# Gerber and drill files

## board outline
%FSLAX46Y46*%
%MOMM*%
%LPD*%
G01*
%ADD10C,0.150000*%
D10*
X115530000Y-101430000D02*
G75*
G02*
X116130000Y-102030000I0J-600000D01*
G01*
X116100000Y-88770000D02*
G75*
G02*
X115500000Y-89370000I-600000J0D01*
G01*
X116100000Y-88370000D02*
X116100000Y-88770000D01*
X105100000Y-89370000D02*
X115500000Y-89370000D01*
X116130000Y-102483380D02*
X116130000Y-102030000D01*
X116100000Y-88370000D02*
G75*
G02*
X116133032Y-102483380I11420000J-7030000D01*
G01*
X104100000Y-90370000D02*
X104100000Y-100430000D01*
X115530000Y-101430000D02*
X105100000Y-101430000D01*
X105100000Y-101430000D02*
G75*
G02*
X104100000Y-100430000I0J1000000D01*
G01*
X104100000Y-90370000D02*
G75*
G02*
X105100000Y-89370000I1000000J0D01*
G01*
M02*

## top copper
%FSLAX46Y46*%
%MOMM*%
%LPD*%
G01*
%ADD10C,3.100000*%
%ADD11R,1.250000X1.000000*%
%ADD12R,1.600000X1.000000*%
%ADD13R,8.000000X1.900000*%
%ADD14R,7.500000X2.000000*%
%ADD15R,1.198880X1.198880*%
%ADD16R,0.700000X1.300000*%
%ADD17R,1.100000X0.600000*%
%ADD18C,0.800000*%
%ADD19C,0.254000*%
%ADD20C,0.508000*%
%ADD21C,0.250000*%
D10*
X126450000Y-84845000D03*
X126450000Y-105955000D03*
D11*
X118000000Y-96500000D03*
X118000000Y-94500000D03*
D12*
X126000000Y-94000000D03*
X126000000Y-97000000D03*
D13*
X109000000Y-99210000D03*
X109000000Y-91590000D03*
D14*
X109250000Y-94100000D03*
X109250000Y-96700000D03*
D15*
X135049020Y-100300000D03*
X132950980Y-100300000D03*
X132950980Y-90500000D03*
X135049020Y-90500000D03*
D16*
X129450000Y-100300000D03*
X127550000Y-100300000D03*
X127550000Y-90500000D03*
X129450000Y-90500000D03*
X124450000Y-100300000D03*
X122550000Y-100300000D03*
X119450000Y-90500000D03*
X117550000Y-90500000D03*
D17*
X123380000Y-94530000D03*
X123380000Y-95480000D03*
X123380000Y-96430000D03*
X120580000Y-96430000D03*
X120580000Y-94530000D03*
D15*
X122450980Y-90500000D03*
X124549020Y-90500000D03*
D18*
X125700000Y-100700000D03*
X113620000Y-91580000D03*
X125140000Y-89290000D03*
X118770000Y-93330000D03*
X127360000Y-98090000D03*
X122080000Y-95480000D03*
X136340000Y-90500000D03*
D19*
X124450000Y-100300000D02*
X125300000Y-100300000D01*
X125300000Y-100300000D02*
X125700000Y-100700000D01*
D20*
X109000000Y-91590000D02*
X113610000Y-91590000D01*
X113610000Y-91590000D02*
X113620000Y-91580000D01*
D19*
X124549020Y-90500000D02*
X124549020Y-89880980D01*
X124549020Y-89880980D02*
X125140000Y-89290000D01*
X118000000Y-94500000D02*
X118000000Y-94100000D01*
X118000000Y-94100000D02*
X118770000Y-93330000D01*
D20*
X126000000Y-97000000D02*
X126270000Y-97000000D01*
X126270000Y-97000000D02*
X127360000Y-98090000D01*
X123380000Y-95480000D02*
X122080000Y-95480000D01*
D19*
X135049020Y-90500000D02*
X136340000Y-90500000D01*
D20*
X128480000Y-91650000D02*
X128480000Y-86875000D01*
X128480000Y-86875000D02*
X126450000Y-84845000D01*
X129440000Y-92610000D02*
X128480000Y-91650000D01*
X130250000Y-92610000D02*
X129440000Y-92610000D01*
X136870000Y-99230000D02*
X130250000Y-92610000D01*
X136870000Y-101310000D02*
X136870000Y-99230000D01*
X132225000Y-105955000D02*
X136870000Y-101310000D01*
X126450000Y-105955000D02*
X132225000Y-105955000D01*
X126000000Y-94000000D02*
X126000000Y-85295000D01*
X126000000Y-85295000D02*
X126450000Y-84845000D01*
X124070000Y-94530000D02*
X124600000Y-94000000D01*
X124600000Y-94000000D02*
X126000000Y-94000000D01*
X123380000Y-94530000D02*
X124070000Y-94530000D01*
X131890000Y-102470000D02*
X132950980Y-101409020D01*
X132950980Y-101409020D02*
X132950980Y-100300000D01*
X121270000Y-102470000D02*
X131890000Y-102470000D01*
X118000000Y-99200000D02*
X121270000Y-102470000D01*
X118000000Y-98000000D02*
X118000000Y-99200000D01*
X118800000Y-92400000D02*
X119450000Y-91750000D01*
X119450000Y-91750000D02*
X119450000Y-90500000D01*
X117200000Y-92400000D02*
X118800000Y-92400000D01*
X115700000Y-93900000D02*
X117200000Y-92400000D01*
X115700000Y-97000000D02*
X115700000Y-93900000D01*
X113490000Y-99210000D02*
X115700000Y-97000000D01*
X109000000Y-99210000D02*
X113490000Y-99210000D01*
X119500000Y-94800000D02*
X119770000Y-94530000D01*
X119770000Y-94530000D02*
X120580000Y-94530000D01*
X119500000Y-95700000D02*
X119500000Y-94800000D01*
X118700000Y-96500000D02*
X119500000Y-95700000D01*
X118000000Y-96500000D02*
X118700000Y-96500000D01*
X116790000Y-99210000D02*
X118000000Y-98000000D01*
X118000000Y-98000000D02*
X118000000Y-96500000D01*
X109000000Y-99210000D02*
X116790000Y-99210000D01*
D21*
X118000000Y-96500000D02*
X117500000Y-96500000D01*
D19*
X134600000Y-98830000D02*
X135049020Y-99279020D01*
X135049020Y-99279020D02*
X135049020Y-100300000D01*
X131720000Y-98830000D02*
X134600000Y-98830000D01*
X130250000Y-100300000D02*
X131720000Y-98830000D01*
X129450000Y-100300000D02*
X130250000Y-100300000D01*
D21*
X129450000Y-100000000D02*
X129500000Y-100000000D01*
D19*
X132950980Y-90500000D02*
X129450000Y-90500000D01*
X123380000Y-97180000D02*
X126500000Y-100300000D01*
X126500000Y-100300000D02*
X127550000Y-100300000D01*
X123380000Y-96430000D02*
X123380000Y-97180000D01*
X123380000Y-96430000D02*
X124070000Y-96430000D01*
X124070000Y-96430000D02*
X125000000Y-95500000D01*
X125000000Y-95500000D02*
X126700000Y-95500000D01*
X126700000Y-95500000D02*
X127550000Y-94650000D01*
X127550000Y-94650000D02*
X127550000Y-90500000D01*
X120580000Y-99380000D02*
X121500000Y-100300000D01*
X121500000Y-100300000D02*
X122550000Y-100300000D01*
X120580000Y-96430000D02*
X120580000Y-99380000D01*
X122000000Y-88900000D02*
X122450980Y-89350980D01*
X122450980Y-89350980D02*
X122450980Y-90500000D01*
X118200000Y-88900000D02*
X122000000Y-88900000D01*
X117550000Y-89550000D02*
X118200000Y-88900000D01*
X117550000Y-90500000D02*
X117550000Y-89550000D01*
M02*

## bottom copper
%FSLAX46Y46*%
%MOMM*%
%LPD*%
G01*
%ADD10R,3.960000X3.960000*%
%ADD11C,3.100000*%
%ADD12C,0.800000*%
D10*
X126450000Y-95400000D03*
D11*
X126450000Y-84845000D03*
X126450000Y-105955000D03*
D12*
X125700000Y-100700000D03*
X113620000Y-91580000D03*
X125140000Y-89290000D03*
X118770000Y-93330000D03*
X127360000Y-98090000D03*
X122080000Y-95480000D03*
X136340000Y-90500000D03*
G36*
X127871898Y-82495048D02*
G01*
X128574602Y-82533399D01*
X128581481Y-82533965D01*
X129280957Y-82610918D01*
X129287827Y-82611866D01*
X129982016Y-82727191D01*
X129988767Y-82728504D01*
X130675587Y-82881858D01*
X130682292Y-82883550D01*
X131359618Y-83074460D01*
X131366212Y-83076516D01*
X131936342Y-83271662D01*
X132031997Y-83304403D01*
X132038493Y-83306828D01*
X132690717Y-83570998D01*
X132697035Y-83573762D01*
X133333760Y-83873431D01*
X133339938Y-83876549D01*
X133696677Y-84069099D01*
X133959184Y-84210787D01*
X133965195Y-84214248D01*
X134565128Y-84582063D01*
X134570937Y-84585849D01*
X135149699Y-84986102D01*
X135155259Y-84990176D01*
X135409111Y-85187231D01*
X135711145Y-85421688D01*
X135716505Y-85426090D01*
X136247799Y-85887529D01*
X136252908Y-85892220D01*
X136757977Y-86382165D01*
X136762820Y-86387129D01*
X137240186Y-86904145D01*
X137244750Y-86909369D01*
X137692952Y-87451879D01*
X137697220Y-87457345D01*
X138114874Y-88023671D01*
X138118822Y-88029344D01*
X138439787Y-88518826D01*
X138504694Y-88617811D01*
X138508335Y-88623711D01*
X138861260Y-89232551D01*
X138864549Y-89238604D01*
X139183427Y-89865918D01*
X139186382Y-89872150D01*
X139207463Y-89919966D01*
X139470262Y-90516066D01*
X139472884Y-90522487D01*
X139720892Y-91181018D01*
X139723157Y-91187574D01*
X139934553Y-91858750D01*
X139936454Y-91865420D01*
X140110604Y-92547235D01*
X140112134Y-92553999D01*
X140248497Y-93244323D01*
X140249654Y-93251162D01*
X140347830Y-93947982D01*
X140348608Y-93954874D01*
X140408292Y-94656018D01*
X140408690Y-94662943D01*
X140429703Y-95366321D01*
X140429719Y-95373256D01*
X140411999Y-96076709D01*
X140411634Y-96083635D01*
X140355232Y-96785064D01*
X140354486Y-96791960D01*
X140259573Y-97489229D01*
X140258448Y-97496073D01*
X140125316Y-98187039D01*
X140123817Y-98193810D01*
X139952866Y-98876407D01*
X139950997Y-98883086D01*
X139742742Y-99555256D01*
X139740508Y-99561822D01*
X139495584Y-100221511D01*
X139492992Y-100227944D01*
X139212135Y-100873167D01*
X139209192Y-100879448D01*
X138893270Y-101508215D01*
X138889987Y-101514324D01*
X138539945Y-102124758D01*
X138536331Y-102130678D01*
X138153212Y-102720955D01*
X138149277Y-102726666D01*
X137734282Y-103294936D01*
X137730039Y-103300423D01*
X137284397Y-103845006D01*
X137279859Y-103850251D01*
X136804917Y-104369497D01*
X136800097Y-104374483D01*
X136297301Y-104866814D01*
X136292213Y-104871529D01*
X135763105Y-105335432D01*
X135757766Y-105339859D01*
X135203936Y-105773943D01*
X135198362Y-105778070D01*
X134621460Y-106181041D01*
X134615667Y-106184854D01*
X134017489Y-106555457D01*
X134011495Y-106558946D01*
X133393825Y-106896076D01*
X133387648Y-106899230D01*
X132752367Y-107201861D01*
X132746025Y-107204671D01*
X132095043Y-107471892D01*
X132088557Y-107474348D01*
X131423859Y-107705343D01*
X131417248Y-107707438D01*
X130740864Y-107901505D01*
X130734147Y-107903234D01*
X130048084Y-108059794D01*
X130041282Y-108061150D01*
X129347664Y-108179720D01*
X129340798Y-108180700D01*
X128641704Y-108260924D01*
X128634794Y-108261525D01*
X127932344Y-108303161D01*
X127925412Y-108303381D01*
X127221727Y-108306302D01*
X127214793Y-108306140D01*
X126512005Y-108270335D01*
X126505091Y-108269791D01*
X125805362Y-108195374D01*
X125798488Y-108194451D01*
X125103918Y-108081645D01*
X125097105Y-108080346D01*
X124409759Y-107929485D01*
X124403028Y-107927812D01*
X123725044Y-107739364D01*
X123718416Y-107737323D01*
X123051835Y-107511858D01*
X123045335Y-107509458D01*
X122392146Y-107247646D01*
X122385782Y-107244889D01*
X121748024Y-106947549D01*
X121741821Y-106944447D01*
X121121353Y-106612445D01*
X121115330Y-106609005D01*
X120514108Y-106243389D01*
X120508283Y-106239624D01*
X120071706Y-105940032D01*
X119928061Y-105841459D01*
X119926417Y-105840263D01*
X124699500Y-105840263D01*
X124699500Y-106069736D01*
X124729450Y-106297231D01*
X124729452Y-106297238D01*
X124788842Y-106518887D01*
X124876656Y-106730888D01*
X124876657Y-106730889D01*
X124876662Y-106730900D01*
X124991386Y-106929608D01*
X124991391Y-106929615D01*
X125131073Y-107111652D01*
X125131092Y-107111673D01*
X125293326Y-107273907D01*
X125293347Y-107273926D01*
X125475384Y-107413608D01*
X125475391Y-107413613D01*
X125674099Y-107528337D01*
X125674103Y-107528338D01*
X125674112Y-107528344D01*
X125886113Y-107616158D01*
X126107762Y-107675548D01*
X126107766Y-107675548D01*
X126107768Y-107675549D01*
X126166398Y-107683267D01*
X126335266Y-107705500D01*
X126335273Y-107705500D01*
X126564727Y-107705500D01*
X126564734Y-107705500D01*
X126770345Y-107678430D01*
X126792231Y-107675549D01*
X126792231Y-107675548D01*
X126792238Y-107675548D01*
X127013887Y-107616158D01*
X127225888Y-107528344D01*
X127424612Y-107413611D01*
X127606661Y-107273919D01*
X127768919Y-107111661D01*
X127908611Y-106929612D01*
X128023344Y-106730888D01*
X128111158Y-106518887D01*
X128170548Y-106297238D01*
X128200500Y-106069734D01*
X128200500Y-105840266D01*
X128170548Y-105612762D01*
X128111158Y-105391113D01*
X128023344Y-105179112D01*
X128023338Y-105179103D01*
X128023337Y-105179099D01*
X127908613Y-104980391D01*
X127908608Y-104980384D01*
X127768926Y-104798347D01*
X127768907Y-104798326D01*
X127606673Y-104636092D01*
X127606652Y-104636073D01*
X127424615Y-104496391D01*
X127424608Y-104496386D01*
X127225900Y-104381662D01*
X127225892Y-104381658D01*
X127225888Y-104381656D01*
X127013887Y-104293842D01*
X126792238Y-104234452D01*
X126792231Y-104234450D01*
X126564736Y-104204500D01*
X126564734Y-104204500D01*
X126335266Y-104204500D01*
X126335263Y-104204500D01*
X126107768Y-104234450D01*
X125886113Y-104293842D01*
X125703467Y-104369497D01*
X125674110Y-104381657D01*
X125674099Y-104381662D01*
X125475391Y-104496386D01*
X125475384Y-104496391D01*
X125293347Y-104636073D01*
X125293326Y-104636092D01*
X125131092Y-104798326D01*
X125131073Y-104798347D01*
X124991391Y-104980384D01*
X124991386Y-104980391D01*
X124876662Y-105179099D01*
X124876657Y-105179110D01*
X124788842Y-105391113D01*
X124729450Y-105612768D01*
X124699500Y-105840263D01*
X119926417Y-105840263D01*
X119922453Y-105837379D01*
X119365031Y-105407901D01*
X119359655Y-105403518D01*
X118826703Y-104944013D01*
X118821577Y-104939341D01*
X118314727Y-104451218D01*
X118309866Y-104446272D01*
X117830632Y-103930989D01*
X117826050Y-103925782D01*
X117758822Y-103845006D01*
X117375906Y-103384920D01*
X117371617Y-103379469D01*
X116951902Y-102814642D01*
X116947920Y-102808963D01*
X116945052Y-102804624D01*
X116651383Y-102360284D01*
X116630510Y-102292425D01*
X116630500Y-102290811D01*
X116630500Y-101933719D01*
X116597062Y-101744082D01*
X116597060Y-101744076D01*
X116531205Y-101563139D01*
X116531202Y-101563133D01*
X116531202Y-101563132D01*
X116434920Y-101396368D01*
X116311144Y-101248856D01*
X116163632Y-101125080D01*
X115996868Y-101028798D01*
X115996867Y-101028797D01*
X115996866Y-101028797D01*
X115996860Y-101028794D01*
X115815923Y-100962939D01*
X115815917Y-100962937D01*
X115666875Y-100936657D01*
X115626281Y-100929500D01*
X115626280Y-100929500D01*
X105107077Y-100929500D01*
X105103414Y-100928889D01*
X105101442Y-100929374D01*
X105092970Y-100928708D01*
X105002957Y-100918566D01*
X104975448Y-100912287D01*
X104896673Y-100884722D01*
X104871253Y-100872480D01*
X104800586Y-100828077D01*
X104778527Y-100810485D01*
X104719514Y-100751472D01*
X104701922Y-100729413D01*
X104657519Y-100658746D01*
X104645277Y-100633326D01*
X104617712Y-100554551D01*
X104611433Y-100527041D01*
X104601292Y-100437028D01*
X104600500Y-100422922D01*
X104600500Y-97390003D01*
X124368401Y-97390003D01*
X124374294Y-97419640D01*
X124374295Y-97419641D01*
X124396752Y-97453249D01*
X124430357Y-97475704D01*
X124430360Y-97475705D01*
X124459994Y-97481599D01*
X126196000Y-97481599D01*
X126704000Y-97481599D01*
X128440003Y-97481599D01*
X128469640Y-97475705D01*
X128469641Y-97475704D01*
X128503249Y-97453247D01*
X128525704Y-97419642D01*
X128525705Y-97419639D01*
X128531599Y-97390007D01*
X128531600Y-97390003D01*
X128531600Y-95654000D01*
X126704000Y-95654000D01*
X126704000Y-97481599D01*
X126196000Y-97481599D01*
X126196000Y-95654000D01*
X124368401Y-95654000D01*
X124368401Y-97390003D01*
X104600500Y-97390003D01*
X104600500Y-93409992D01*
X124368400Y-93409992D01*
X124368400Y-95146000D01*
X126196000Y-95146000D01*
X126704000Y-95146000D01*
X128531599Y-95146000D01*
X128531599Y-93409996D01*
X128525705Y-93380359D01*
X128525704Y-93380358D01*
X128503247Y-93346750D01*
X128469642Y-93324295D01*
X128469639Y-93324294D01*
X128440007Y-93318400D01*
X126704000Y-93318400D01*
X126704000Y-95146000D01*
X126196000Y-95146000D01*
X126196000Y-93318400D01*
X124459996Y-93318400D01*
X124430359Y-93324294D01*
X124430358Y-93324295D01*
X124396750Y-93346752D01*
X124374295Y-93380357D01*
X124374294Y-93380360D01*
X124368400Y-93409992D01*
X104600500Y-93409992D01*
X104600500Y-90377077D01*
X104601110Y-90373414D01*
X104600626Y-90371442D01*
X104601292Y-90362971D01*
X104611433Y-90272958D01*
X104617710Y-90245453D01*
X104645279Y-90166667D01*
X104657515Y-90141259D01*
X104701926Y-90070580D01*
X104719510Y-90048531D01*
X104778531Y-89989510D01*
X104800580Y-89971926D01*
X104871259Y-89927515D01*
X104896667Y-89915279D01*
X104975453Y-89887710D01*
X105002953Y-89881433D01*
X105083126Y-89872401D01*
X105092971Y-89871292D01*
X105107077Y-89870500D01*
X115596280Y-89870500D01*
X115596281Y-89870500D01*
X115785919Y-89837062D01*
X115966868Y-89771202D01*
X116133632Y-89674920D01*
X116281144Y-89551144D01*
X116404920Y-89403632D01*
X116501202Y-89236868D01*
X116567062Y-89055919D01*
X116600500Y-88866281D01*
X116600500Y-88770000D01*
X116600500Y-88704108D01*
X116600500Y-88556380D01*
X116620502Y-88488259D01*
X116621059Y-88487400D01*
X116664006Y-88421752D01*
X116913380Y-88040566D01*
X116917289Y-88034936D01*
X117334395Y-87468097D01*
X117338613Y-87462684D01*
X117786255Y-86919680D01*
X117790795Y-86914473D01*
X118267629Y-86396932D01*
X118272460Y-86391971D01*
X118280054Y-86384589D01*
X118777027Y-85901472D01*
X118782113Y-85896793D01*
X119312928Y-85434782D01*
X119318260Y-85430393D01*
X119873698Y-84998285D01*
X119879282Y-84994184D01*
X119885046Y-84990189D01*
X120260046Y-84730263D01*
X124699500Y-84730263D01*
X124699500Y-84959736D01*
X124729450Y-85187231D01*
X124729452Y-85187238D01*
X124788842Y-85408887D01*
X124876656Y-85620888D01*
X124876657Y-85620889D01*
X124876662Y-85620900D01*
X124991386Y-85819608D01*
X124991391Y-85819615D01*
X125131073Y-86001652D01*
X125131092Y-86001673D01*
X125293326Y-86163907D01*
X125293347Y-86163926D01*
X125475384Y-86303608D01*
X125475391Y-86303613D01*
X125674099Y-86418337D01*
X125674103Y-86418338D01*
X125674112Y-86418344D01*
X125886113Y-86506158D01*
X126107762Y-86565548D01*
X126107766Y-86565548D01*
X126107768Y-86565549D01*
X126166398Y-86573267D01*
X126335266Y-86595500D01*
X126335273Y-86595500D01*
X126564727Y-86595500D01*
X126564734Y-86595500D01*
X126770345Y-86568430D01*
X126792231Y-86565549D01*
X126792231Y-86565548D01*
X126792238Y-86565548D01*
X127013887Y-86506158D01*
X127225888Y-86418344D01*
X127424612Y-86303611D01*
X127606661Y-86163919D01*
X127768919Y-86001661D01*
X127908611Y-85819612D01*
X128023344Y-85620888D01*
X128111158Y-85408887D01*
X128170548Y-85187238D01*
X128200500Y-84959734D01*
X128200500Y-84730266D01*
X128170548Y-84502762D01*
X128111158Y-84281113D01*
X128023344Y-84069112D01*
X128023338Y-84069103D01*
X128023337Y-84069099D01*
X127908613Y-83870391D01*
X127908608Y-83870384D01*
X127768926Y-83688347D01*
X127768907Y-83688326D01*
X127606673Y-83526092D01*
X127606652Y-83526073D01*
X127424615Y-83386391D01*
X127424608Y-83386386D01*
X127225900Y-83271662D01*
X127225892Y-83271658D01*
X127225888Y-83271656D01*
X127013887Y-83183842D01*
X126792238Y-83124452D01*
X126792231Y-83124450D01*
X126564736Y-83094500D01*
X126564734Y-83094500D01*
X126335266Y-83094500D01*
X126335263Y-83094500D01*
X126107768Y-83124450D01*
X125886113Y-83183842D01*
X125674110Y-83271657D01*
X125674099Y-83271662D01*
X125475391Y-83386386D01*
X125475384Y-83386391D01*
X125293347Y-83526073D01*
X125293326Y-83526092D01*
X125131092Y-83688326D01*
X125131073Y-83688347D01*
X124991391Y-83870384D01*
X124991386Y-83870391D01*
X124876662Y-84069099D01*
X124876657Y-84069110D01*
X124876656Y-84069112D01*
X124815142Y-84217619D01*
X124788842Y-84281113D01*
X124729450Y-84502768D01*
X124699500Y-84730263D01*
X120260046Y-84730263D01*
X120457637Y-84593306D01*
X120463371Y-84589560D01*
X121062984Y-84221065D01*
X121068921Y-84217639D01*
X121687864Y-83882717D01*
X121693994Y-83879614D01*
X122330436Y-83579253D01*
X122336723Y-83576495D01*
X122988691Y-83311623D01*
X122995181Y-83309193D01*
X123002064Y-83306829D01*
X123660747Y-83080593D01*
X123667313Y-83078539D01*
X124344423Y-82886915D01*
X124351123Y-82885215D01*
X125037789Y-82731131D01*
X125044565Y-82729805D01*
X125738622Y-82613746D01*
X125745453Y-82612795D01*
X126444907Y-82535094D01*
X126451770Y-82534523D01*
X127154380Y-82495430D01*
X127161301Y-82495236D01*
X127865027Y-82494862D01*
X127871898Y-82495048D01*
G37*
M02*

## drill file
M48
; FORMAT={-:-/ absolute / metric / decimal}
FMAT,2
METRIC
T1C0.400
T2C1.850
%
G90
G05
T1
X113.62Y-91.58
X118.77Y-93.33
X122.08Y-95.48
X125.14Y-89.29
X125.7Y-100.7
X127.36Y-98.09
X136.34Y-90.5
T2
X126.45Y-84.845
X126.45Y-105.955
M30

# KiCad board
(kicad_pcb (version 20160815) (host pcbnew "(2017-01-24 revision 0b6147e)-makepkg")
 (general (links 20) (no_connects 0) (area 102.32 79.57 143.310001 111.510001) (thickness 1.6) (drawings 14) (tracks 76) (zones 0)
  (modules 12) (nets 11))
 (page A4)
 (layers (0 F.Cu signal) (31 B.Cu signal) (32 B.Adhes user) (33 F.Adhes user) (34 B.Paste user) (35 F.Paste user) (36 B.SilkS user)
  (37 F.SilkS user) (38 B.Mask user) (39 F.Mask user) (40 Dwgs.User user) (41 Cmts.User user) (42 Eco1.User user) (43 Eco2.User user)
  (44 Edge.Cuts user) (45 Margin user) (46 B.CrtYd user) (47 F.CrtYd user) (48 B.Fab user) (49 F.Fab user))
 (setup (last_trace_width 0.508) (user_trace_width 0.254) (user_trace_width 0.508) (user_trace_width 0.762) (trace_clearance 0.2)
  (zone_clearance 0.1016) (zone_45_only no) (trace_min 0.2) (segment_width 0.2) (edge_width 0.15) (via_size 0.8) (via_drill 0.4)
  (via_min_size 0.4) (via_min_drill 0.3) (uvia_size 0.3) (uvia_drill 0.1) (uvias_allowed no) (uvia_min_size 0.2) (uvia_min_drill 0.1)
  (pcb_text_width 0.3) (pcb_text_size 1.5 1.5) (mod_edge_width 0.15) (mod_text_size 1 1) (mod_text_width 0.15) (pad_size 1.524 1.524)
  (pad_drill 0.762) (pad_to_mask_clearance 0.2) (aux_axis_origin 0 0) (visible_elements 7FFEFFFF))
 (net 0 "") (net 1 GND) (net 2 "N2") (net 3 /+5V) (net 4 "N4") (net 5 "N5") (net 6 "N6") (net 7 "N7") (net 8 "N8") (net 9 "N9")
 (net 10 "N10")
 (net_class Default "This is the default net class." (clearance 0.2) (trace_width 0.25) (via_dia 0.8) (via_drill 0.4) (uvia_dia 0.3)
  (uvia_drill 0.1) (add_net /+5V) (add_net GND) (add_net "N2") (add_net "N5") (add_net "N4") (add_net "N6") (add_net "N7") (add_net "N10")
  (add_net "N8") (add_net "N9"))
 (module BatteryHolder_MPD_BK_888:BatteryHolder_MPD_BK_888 (layer B.Cu) (at 126.45 95.4 90)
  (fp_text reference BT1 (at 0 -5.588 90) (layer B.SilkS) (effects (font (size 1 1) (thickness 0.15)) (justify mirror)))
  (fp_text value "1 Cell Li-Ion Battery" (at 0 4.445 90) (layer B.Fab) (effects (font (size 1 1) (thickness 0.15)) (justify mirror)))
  (pad 2 smd rect (at 0 0 90) (size 3.96 3.96) (layers B.Cu B.Paste B.Mask) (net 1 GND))
  (pad 1 thru_hole circle (at 10.555 0 90) (size 3.1 3.1) (drill 1.85) (layers *.Cu *.Mask) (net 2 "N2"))
  (pad 1 thru_hole circle (at -10.555 0 90) (size 3.1 3.1) (drill 1.85) (layers *.Cu *.Mask) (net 2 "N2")))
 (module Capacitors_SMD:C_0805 (layer F.Cu) (at 118 95.5 90)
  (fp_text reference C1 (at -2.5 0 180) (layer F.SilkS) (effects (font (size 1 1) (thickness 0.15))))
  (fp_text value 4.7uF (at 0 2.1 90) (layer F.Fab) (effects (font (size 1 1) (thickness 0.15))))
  (pad 1 smd rect (at -1 0 90) (size 1 1.25) (layers F.Cu F.Paste F.Mask) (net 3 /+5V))
  (pad 2 smd rect (at 1 0 90) (size 1 1.25) (layers F.Cu F.Paste F.Mask) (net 1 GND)))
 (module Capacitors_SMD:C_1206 (layer F.Cu) (at 126 95.5 270)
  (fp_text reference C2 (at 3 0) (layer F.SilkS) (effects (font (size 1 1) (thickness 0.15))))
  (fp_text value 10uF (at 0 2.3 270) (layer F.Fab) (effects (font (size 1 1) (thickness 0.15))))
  (pad 1 smd rect (at -1.5 0 270) (size 1 1.6) (layers F.Cu F.Paste F.Mask) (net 2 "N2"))
  (pad 2 smd rect (at 1.5 0 270) (size 1 1.6) (layers F.Cu F.Paste F.Mask) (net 1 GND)))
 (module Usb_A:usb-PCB (layer F.Cu) (at 104.1 95.4 270)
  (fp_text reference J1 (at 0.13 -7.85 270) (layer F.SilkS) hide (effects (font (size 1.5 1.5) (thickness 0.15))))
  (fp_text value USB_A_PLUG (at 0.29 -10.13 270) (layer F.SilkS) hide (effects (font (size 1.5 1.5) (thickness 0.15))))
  (pad 1 connect rect (at 3.81 -4.9 270) (size 1.9 8) (layers F.Cu F.Mask) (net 3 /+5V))
  (pad 4 connect rect (at -3.81 -4.9 270) (size 1.9 8) (layers F.Cu F.Mask) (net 1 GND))
  (pad 3 connect rect (at -1.3 -5.15 270) (size 2 7.5) (layers F.Cu F.Mask) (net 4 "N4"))
  (pad 2 connect rect (at 1.3 -5.15 270) (size 2 7.5) (layers F.Cu F.Mask) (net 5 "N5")))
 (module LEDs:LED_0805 (layer F.Cu) (at 134 100.3 180)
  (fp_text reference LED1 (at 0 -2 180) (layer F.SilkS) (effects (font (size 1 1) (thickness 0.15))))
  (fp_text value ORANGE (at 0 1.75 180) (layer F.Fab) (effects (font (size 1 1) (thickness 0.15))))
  (pad 1 smd rect (at -1.04902 0) (size 1.19888 1.19888) (layers F.Cu F.Paste F.Mask) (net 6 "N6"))
  (pad 2 smd rect (at 1.04902 0) (size 1.19888 1.19888) (layers F.Cu F.Paste F.Mask) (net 3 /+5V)))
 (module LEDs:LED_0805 (layer F.Cu) (at 134 90.5 180)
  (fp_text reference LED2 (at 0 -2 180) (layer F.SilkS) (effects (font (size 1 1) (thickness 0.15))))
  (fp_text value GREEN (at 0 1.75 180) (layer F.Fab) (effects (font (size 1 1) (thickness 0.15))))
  (pad 2 smd rect (at 1.04902 0) (size 1.19888 1.19888) (layers F.Cu F.Paste F.Mask) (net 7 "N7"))
  (pad 1 smd rect (at -1.04902 0) (size 1.19888 1.19888) (layers F.Cu F.Paste F.Mask) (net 1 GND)))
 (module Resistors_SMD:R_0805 (layer F.Cu) (at 128.5 100.3 180)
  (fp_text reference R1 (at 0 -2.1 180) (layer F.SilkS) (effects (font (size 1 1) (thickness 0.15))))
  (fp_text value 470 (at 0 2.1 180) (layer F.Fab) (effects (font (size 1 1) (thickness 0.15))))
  (pad 1 smd rect (at -0.95 0 180) (size 0.7 1.3) (layers F.Cu F.Paste F.Mask) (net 6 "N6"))
  (pad 2 smd rect (at 0.95 0 180) (size 0.7 1.3) (layers F.Cu F.Paste F.Mask) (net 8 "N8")))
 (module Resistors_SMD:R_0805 (layer F.Cu) (at 128.5 90.5 180)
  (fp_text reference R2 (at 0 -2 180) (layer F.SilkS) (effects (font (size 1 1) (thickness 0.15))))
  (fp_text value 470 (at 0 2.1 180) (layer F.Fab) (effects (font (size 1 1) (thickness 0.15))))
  (pad 2 smd rect (at 0.95 0 180) (size 0.7 1.3) (layers F.Cu F.Paste F.Mask) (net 8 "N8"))
  (pad 1 smd rect (at -0.95 0 180) (size 0.7 1.3) (layers F.Cu F.Paste F.Mask) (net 7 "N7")))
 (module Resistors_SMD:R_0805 (layer F.Cu) (at 123.5 100.3)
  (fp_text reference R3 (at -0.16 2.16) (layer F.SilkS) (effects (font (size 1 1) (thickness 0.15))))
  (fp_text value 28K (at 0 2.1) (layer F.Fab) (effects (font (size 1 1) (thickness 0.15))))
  (pad 2 smd rect (at 0.95 0) (size 0.7 1.3) (layers F.Cu F.Paste F.Mask) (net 1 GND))
  (pad 1 smd rect (at -0.95 0) (size 0.7 1.3) (layers F.Cu F.Paste F.Mask) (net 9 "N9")))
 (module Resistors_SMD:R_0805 (layer F.Cu) (at 118.5 90.5 180)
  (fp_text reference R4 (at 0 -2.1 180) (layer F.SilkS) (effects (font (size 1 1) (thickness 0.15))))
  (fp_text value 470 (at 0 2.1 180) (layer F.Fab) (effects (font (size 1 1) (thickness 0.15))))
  (pad 1 smd rect (at -0.95 0 180) (size 0.7 1.3) (layers F.Cu F.Paste F.Mask) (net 3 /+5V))
  (pad 2 smd rect (at 0.95 0 180) (size 0.7 1.3) (layers F.Cu F.Paste F.Mask) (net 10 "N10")))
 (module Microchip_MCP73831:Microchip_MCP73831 (layer F.Cu) (at 122 95.5 90)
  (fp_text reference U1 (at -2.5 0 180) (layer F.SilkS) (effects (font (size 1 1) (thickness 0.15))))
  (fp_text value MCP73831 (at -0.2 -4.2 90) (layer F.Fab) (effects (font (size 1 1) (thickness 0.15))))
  (pad 3 smd rect (at 0.97 1.38 90) (size 0.6 1.1) (layers F.Cu F.Paste F.Mask) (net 2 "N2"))
  (pad 2 smd rect (at 0.02 1.38 90) (size 0.6 1.1) (layers F.Cu F.Paste F.Mask) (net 1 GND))
  (pad 1 smd rect (at -0.93 1.38 90) (size 0.6 1.1) (layers F.Cu F.Paste F.Mask) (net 8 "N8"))
  (pad 5 smd rect (at -0.93 -1.42 90) (size 0.6 1.1) (layers F.Cu F.Paste F.Mask) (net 9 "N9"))
  (pad 4 smd rect (at 0.97 -1.42 90) (size 0.6 1.1) (layers F.Cu F.Paste F.Mask) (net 3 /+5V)))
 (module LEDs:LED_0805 (layer F.Cu) (at 123.5 90.5 180)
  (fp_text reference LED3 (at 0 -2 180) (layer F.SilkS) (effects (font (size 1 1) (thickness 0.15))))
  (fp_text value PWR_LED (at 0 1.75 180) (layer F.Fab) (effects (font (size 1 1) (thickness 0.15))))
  (pad 2 smd rect (at 1.04902 0) (size 1.19888 1.19888) (layers F.Cu F.Paste F.Mask) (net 10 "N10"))
  (pad 1 smd rect (at -1.04902 0) (size 1.19888 1.19888) (layers F.Cu F.Paste F.Mask) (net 1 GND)))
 (gr_arc (start 115.53 102.03) (end 116.13 102.03) (angle -90) (layer Edge.Cuts) (width 0.15))
 (gr_arc (start 115.5 88.77) (end 116.1 88.77) (angle 90) (layer Edge.Cuts) (width 0.15))
 (gr_line (start 116.1 88.37) (end 116.1 88.77) (angle 90) (layer Edge.Cuts) (width 0.15))
 (gr_line (start 105.1 89.37) (end 115.5 89.37) (angle 90) (layer Edge.Cuts) (width 0.15))
 (gr_line (start 116.13 102.48338) (end 116.13 102.03) (angle 90) (layer Edge.Cuts) (width 0.15))
 (gr_arc (start 127.52 95.4) (end 116.1 88.37) (angle 296.5) (layer Edge.Cuts) (width 0.15))
 (gr_line (start 104.1 90.37) (end 104.1 100.43) (angle 90) (layer Edge.Cuts) (width 0.15))
 (gr_line (start 115.53 101.43) (end 105.1 101.43) (angle 90) (layer Edge.Cuts) (width 0.15))
 (gr_arc (start 105.1 100.43) (end 105.1 101.43) (angle 90) (layer Edge.Cuts) (width 0.15))
 (gr_arc (start 105.1 90.37) (end 104.1 90.37) (angle 90) (layer Edge.Cuts) (width 0.15))
 (segment (start 124.45 100.3) (end 125.3 100.3) (width 0.254) (layer F.Cu) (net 1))
 (segment (start 125.3 100.3) (end 125.7 100.7) (width 0.254) (layer F.Cu) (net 1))
 (via (at 125.7 100.7) (size 0.8) (drill 0.4) (layers F.Cu B.Cu) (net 1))
 (segment (start 109 91.59) (end 113.61 91.59) (width 0.508) (layer F.Cu) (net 1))
 (segment (start 113.61 91.59) (end 113.62 91.58) (width 0.508) (layer F.Cu) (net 1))
 (via (at 113.62 91.58) (size 0.8) (drill 0.4) (layers F.Cu B.Cu) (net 1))
 (segment (start 124.54902 90.5) (end 124.54902 89.88098) (width 0.254) (layer F.Cu) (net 1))
 (segment (start 124.54902 89.88098) (end 125.14 89.29) (width 0.254) (layer F.Cu) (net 1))
 (via (at 125.14 89.29) (size 0.8) (drill 0.4) (layers F.Cu B.Cu) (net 1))
 (segment (start 118 94.5) (end 118 94.1) (width 0.254) (layer F.Cu) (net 1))
 (segment (start 118 94.1) (end 118.77 93.33) (width 0.254) (layer F.Cu) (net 1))
 (via (at 118.77 93.33) (size 0.8) (drill 0.4) (layers F.Cu B.Cu) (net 1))
 (segment (start 126 97) (end 126.27 97) (width 0.508) (layer F.Cu) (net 1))
 (segment (start 126.27 97) (end 127.36 98.09) (width 0.508) (layer F.Cu) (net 1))
 (via (at 127.36 98.09) (size 0.8) (drill 0.4) (layers F.Cu B.Cu) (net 1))
 (segment (start 123.38 95.48) (end 122.08 95.48) (width 0.508) (layer F.Cu) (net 1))
 (via (at 122.08 95.48) (size 0.8) (drill 0.4) (layers F.Cu B.Cu) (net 1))
 (segment (start 135.04902 90.5) (end 136.34 90.5) (width 0.254) (layer F.Cu) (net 1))
 (via (at 136.34 90.5) (size 0.8) (drill 0.4) (layers F.Cu B.Cu) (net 1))
 (segment (start 128.48 91.65) (end 128.48 86.875) (width 0.508) (layer F.Cu) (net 2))
 (segment (start 128.48 86.875) (end 126.45 84.845) (width 0.508) (layer F.Cu) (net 2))
 (segment (start 129.44 92.61) (end 128.48 91.65) (width 0.508) (layer F.Cu) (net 2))
 (segment (start 130.25 92.61) (end 129.44 92.61) (width 0.508) (layer F.Cu) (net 2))
 (segment (start 136.87 99.23) (end 130.25 92.61) (width 0.508) (layer F.Cu) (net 2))
 (segment (start 136.87 101.31) (end 136.87 99.23) (width 0.508) (layer F.Cu) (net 2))
 (segment (start 132.225 105.955) (end 136.87 101.31) (width 0.508) (layer F.Cu) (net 2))
 (segment (start 126.45 105.955) (end 132.225 105.955) (width 0.508) (layer F.Cu) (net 2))
 (segment (start 126 94) (end 126 85.295) (width 0.508) (layer F.Cu) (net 2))
 (segment (start 126 85.295) (end 126.45 84.845) (width 0.508) (layer F.Cu) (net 2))
 (segment (start 124.07 94.53) (end 124.6 94) (width 0.508) (layer F.Cu) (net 2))
 (segment (start 124.6 94) (end 126 94) (width 0.508) (layer F.Cu) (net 2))
 (segment (start 123.38 94.53) (end 124.07 94.53) (width 0.508) (layer F.Cu) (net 2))
 (segment (start 131.89 102.47) (end 132.95098 101.40902) (width 0.508) (layer F.Cu) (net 3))
 (segment (start 132.95098 101.40902) (end 132.95098 100.3) (width 0.508) (layer F.Cu) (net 3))
 (segment (start 121.27 102.47) (end 131.89 102.47) (width 0.508) (layer F.Cu) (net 3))
 (segment (start 118 99.2) (end 121.27 102.47) (width 0.508) (layer F.Cu) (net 3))
 (segment (start 118 98) (end 118 99.2) (width 0.508) (layer F.Cu) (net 3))
 (segment (start 118.8 92.4) (end 119.45 91.75) (width 0.508) (layer F.Cu) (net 3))
 (segment (start 119.45 91.75) (end 119.45 90.5) (width 0.508) (layer F.Cu) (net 3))
 (segment (start 117.2 92.4) (end 118.8 92.4) (width 0.508) (layer F.Cu) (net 3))
 (segment (start 115.7 93.9) (end 117.2 92.4) (width 0.508) (layer F.Cu) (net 3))
 (segment (start 115.7 97) (end 115.7 93.9) (width 0.508) (layer F.Cu) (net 3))
 (segment (start 113.49 99.21) (end 115.7 97) (width 0.508) (layer F.Cu) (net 3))
 (segment (start 109 99.21) (end 113.49 99.21) (width 0.508) (layer F.Cu) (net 3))
 (segment (start 119.5 94.8) (end 119.77 94.53) (width 0.508) (layer F.Cu) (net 3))
 (segment (start 119.77 94.53) (end 120.58 94.53) (width 0.508) (layer F.Cu) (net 3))
 (segment (start 119.5 95.7) (end 119.5 94.8) (width 0.508) (layer F.Cu) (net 3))
 (segment (start 118.7 96.5) (end 119.5 95.7) (width 0.508) (layer F.Cu) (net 3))
 (segment (start 118 96.5) (end 118.7 96.5) (width 0.508) (layer F.Cu) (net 3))
 (segment (start 116.79 99.21) (end 118 98) (width 0.508) (layer F.Cu) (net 3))
 (segment (start 118 98) (end 118 96.5) (width 0.508) (layer F.Cu) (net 3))
 (segment (start 109 99.21) (end 116.79 99.21) (width 0.508) (layer F.Cu) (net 3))
 (segment (start 118 96.5) (end 117.5 96.5) (width 0.25) (layer F.Cu) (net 3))
 (segment (start 134.6 98.83) (end 135.04902 99.27902) (width 0.254) (layer F.Cu) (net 6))
 (segment (start 135.04902 99.27902) (end 135.04902 100.3) (width 0.254) (layer F.Cu) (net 6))
 (segment (start 131.72 98.83) (end 134.6 98.83) (width 0.254) (layer F.Cu) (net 6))
 (segment (start 130.25 100.3) (end 131.72 98.83) (width 0.254) (layer F.Cu) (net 6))
 (segment (start 129.45 100.3) (end 130.25 100.3) (width 0.254) (layer F.Cu) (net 6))
 (segment (start 129.45 100) (end 129.5 100) (width 0.25) (layer F.Cu) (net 6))
 (segment (start 132.95098 90.5) (end 129.45 90.5) (width 0.254) (layer F.Cu) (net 7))
 (segment (start 123.38 97.18) (end 126.5 100.3) (width 0.254) (layer F.Cu) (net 8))
 (segment (start 126.5 100.3) (end 127.55 100.3) (width 0.254) (layer F.Cu) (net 8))
 (segment (start 123.38 96.43) (end 123.38 97.18) (width 0.254) (layer F.Cu) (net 8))
 (segment (start 123.38 96.43) (end 124.07 96.43) (width 0.254) (layer F.Cu) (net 8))
 (segment (start 124.07 96.43) (end 125 95.5) (width 0.254) (layer F.Cu) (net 8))
 (segment (start 125 95.5) (end 126.7 95.5) (width 0.254) (layer F.Cu) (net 8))
 (segment (start 126.7 95.5) (end 127.55 94.65) (width 0.254) (layer F.Cu) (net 8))
 (segment (start 127.55 94.65) (end 127.55 90.5) (width 0.254) (layer F.Cu) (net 8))
 (segment (start 120.58 99.38) (end 121.5 100.3) (width 0.254) (layer F.Cu) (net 9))
 (segment (start 121.5 100.3) (end 122.55 100.3) (width 0.254) (layer F.Cu) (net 9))
 (segment (start 120.58 96.43) (end 120.58 99.38) (width 0.254) (layer F.Cu) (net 9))
 (segment (start 122 88.9) (end 122.45098 89.35098) (width 0.254) (layer F.Cu) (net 10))
 (segment (start 122.45098 89.35098) (end 122.45098 90.5) (width 0.254) (layer F.Cu) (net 10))
 (segment (start 118.2 88.9) (end 122 88.9) (width 0.254) (layer F.Cu) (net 10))
 (segment (start 117.55 89.55) (end 118.2 88.9) (width 0.254) (layer F.Cu) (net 10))
 (segment (start 117.55 90.5) (end 117.55 89.55) (width 0.254) (layer F.Cu) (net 10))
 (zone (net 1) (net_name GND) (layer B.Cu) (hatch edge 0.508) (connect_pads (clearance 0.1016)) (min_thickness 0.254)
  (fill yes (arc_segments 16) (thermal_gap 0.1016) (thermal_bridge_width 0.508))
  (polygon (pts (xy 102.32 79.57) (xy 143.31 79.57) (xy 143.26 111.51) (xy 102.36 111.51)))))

